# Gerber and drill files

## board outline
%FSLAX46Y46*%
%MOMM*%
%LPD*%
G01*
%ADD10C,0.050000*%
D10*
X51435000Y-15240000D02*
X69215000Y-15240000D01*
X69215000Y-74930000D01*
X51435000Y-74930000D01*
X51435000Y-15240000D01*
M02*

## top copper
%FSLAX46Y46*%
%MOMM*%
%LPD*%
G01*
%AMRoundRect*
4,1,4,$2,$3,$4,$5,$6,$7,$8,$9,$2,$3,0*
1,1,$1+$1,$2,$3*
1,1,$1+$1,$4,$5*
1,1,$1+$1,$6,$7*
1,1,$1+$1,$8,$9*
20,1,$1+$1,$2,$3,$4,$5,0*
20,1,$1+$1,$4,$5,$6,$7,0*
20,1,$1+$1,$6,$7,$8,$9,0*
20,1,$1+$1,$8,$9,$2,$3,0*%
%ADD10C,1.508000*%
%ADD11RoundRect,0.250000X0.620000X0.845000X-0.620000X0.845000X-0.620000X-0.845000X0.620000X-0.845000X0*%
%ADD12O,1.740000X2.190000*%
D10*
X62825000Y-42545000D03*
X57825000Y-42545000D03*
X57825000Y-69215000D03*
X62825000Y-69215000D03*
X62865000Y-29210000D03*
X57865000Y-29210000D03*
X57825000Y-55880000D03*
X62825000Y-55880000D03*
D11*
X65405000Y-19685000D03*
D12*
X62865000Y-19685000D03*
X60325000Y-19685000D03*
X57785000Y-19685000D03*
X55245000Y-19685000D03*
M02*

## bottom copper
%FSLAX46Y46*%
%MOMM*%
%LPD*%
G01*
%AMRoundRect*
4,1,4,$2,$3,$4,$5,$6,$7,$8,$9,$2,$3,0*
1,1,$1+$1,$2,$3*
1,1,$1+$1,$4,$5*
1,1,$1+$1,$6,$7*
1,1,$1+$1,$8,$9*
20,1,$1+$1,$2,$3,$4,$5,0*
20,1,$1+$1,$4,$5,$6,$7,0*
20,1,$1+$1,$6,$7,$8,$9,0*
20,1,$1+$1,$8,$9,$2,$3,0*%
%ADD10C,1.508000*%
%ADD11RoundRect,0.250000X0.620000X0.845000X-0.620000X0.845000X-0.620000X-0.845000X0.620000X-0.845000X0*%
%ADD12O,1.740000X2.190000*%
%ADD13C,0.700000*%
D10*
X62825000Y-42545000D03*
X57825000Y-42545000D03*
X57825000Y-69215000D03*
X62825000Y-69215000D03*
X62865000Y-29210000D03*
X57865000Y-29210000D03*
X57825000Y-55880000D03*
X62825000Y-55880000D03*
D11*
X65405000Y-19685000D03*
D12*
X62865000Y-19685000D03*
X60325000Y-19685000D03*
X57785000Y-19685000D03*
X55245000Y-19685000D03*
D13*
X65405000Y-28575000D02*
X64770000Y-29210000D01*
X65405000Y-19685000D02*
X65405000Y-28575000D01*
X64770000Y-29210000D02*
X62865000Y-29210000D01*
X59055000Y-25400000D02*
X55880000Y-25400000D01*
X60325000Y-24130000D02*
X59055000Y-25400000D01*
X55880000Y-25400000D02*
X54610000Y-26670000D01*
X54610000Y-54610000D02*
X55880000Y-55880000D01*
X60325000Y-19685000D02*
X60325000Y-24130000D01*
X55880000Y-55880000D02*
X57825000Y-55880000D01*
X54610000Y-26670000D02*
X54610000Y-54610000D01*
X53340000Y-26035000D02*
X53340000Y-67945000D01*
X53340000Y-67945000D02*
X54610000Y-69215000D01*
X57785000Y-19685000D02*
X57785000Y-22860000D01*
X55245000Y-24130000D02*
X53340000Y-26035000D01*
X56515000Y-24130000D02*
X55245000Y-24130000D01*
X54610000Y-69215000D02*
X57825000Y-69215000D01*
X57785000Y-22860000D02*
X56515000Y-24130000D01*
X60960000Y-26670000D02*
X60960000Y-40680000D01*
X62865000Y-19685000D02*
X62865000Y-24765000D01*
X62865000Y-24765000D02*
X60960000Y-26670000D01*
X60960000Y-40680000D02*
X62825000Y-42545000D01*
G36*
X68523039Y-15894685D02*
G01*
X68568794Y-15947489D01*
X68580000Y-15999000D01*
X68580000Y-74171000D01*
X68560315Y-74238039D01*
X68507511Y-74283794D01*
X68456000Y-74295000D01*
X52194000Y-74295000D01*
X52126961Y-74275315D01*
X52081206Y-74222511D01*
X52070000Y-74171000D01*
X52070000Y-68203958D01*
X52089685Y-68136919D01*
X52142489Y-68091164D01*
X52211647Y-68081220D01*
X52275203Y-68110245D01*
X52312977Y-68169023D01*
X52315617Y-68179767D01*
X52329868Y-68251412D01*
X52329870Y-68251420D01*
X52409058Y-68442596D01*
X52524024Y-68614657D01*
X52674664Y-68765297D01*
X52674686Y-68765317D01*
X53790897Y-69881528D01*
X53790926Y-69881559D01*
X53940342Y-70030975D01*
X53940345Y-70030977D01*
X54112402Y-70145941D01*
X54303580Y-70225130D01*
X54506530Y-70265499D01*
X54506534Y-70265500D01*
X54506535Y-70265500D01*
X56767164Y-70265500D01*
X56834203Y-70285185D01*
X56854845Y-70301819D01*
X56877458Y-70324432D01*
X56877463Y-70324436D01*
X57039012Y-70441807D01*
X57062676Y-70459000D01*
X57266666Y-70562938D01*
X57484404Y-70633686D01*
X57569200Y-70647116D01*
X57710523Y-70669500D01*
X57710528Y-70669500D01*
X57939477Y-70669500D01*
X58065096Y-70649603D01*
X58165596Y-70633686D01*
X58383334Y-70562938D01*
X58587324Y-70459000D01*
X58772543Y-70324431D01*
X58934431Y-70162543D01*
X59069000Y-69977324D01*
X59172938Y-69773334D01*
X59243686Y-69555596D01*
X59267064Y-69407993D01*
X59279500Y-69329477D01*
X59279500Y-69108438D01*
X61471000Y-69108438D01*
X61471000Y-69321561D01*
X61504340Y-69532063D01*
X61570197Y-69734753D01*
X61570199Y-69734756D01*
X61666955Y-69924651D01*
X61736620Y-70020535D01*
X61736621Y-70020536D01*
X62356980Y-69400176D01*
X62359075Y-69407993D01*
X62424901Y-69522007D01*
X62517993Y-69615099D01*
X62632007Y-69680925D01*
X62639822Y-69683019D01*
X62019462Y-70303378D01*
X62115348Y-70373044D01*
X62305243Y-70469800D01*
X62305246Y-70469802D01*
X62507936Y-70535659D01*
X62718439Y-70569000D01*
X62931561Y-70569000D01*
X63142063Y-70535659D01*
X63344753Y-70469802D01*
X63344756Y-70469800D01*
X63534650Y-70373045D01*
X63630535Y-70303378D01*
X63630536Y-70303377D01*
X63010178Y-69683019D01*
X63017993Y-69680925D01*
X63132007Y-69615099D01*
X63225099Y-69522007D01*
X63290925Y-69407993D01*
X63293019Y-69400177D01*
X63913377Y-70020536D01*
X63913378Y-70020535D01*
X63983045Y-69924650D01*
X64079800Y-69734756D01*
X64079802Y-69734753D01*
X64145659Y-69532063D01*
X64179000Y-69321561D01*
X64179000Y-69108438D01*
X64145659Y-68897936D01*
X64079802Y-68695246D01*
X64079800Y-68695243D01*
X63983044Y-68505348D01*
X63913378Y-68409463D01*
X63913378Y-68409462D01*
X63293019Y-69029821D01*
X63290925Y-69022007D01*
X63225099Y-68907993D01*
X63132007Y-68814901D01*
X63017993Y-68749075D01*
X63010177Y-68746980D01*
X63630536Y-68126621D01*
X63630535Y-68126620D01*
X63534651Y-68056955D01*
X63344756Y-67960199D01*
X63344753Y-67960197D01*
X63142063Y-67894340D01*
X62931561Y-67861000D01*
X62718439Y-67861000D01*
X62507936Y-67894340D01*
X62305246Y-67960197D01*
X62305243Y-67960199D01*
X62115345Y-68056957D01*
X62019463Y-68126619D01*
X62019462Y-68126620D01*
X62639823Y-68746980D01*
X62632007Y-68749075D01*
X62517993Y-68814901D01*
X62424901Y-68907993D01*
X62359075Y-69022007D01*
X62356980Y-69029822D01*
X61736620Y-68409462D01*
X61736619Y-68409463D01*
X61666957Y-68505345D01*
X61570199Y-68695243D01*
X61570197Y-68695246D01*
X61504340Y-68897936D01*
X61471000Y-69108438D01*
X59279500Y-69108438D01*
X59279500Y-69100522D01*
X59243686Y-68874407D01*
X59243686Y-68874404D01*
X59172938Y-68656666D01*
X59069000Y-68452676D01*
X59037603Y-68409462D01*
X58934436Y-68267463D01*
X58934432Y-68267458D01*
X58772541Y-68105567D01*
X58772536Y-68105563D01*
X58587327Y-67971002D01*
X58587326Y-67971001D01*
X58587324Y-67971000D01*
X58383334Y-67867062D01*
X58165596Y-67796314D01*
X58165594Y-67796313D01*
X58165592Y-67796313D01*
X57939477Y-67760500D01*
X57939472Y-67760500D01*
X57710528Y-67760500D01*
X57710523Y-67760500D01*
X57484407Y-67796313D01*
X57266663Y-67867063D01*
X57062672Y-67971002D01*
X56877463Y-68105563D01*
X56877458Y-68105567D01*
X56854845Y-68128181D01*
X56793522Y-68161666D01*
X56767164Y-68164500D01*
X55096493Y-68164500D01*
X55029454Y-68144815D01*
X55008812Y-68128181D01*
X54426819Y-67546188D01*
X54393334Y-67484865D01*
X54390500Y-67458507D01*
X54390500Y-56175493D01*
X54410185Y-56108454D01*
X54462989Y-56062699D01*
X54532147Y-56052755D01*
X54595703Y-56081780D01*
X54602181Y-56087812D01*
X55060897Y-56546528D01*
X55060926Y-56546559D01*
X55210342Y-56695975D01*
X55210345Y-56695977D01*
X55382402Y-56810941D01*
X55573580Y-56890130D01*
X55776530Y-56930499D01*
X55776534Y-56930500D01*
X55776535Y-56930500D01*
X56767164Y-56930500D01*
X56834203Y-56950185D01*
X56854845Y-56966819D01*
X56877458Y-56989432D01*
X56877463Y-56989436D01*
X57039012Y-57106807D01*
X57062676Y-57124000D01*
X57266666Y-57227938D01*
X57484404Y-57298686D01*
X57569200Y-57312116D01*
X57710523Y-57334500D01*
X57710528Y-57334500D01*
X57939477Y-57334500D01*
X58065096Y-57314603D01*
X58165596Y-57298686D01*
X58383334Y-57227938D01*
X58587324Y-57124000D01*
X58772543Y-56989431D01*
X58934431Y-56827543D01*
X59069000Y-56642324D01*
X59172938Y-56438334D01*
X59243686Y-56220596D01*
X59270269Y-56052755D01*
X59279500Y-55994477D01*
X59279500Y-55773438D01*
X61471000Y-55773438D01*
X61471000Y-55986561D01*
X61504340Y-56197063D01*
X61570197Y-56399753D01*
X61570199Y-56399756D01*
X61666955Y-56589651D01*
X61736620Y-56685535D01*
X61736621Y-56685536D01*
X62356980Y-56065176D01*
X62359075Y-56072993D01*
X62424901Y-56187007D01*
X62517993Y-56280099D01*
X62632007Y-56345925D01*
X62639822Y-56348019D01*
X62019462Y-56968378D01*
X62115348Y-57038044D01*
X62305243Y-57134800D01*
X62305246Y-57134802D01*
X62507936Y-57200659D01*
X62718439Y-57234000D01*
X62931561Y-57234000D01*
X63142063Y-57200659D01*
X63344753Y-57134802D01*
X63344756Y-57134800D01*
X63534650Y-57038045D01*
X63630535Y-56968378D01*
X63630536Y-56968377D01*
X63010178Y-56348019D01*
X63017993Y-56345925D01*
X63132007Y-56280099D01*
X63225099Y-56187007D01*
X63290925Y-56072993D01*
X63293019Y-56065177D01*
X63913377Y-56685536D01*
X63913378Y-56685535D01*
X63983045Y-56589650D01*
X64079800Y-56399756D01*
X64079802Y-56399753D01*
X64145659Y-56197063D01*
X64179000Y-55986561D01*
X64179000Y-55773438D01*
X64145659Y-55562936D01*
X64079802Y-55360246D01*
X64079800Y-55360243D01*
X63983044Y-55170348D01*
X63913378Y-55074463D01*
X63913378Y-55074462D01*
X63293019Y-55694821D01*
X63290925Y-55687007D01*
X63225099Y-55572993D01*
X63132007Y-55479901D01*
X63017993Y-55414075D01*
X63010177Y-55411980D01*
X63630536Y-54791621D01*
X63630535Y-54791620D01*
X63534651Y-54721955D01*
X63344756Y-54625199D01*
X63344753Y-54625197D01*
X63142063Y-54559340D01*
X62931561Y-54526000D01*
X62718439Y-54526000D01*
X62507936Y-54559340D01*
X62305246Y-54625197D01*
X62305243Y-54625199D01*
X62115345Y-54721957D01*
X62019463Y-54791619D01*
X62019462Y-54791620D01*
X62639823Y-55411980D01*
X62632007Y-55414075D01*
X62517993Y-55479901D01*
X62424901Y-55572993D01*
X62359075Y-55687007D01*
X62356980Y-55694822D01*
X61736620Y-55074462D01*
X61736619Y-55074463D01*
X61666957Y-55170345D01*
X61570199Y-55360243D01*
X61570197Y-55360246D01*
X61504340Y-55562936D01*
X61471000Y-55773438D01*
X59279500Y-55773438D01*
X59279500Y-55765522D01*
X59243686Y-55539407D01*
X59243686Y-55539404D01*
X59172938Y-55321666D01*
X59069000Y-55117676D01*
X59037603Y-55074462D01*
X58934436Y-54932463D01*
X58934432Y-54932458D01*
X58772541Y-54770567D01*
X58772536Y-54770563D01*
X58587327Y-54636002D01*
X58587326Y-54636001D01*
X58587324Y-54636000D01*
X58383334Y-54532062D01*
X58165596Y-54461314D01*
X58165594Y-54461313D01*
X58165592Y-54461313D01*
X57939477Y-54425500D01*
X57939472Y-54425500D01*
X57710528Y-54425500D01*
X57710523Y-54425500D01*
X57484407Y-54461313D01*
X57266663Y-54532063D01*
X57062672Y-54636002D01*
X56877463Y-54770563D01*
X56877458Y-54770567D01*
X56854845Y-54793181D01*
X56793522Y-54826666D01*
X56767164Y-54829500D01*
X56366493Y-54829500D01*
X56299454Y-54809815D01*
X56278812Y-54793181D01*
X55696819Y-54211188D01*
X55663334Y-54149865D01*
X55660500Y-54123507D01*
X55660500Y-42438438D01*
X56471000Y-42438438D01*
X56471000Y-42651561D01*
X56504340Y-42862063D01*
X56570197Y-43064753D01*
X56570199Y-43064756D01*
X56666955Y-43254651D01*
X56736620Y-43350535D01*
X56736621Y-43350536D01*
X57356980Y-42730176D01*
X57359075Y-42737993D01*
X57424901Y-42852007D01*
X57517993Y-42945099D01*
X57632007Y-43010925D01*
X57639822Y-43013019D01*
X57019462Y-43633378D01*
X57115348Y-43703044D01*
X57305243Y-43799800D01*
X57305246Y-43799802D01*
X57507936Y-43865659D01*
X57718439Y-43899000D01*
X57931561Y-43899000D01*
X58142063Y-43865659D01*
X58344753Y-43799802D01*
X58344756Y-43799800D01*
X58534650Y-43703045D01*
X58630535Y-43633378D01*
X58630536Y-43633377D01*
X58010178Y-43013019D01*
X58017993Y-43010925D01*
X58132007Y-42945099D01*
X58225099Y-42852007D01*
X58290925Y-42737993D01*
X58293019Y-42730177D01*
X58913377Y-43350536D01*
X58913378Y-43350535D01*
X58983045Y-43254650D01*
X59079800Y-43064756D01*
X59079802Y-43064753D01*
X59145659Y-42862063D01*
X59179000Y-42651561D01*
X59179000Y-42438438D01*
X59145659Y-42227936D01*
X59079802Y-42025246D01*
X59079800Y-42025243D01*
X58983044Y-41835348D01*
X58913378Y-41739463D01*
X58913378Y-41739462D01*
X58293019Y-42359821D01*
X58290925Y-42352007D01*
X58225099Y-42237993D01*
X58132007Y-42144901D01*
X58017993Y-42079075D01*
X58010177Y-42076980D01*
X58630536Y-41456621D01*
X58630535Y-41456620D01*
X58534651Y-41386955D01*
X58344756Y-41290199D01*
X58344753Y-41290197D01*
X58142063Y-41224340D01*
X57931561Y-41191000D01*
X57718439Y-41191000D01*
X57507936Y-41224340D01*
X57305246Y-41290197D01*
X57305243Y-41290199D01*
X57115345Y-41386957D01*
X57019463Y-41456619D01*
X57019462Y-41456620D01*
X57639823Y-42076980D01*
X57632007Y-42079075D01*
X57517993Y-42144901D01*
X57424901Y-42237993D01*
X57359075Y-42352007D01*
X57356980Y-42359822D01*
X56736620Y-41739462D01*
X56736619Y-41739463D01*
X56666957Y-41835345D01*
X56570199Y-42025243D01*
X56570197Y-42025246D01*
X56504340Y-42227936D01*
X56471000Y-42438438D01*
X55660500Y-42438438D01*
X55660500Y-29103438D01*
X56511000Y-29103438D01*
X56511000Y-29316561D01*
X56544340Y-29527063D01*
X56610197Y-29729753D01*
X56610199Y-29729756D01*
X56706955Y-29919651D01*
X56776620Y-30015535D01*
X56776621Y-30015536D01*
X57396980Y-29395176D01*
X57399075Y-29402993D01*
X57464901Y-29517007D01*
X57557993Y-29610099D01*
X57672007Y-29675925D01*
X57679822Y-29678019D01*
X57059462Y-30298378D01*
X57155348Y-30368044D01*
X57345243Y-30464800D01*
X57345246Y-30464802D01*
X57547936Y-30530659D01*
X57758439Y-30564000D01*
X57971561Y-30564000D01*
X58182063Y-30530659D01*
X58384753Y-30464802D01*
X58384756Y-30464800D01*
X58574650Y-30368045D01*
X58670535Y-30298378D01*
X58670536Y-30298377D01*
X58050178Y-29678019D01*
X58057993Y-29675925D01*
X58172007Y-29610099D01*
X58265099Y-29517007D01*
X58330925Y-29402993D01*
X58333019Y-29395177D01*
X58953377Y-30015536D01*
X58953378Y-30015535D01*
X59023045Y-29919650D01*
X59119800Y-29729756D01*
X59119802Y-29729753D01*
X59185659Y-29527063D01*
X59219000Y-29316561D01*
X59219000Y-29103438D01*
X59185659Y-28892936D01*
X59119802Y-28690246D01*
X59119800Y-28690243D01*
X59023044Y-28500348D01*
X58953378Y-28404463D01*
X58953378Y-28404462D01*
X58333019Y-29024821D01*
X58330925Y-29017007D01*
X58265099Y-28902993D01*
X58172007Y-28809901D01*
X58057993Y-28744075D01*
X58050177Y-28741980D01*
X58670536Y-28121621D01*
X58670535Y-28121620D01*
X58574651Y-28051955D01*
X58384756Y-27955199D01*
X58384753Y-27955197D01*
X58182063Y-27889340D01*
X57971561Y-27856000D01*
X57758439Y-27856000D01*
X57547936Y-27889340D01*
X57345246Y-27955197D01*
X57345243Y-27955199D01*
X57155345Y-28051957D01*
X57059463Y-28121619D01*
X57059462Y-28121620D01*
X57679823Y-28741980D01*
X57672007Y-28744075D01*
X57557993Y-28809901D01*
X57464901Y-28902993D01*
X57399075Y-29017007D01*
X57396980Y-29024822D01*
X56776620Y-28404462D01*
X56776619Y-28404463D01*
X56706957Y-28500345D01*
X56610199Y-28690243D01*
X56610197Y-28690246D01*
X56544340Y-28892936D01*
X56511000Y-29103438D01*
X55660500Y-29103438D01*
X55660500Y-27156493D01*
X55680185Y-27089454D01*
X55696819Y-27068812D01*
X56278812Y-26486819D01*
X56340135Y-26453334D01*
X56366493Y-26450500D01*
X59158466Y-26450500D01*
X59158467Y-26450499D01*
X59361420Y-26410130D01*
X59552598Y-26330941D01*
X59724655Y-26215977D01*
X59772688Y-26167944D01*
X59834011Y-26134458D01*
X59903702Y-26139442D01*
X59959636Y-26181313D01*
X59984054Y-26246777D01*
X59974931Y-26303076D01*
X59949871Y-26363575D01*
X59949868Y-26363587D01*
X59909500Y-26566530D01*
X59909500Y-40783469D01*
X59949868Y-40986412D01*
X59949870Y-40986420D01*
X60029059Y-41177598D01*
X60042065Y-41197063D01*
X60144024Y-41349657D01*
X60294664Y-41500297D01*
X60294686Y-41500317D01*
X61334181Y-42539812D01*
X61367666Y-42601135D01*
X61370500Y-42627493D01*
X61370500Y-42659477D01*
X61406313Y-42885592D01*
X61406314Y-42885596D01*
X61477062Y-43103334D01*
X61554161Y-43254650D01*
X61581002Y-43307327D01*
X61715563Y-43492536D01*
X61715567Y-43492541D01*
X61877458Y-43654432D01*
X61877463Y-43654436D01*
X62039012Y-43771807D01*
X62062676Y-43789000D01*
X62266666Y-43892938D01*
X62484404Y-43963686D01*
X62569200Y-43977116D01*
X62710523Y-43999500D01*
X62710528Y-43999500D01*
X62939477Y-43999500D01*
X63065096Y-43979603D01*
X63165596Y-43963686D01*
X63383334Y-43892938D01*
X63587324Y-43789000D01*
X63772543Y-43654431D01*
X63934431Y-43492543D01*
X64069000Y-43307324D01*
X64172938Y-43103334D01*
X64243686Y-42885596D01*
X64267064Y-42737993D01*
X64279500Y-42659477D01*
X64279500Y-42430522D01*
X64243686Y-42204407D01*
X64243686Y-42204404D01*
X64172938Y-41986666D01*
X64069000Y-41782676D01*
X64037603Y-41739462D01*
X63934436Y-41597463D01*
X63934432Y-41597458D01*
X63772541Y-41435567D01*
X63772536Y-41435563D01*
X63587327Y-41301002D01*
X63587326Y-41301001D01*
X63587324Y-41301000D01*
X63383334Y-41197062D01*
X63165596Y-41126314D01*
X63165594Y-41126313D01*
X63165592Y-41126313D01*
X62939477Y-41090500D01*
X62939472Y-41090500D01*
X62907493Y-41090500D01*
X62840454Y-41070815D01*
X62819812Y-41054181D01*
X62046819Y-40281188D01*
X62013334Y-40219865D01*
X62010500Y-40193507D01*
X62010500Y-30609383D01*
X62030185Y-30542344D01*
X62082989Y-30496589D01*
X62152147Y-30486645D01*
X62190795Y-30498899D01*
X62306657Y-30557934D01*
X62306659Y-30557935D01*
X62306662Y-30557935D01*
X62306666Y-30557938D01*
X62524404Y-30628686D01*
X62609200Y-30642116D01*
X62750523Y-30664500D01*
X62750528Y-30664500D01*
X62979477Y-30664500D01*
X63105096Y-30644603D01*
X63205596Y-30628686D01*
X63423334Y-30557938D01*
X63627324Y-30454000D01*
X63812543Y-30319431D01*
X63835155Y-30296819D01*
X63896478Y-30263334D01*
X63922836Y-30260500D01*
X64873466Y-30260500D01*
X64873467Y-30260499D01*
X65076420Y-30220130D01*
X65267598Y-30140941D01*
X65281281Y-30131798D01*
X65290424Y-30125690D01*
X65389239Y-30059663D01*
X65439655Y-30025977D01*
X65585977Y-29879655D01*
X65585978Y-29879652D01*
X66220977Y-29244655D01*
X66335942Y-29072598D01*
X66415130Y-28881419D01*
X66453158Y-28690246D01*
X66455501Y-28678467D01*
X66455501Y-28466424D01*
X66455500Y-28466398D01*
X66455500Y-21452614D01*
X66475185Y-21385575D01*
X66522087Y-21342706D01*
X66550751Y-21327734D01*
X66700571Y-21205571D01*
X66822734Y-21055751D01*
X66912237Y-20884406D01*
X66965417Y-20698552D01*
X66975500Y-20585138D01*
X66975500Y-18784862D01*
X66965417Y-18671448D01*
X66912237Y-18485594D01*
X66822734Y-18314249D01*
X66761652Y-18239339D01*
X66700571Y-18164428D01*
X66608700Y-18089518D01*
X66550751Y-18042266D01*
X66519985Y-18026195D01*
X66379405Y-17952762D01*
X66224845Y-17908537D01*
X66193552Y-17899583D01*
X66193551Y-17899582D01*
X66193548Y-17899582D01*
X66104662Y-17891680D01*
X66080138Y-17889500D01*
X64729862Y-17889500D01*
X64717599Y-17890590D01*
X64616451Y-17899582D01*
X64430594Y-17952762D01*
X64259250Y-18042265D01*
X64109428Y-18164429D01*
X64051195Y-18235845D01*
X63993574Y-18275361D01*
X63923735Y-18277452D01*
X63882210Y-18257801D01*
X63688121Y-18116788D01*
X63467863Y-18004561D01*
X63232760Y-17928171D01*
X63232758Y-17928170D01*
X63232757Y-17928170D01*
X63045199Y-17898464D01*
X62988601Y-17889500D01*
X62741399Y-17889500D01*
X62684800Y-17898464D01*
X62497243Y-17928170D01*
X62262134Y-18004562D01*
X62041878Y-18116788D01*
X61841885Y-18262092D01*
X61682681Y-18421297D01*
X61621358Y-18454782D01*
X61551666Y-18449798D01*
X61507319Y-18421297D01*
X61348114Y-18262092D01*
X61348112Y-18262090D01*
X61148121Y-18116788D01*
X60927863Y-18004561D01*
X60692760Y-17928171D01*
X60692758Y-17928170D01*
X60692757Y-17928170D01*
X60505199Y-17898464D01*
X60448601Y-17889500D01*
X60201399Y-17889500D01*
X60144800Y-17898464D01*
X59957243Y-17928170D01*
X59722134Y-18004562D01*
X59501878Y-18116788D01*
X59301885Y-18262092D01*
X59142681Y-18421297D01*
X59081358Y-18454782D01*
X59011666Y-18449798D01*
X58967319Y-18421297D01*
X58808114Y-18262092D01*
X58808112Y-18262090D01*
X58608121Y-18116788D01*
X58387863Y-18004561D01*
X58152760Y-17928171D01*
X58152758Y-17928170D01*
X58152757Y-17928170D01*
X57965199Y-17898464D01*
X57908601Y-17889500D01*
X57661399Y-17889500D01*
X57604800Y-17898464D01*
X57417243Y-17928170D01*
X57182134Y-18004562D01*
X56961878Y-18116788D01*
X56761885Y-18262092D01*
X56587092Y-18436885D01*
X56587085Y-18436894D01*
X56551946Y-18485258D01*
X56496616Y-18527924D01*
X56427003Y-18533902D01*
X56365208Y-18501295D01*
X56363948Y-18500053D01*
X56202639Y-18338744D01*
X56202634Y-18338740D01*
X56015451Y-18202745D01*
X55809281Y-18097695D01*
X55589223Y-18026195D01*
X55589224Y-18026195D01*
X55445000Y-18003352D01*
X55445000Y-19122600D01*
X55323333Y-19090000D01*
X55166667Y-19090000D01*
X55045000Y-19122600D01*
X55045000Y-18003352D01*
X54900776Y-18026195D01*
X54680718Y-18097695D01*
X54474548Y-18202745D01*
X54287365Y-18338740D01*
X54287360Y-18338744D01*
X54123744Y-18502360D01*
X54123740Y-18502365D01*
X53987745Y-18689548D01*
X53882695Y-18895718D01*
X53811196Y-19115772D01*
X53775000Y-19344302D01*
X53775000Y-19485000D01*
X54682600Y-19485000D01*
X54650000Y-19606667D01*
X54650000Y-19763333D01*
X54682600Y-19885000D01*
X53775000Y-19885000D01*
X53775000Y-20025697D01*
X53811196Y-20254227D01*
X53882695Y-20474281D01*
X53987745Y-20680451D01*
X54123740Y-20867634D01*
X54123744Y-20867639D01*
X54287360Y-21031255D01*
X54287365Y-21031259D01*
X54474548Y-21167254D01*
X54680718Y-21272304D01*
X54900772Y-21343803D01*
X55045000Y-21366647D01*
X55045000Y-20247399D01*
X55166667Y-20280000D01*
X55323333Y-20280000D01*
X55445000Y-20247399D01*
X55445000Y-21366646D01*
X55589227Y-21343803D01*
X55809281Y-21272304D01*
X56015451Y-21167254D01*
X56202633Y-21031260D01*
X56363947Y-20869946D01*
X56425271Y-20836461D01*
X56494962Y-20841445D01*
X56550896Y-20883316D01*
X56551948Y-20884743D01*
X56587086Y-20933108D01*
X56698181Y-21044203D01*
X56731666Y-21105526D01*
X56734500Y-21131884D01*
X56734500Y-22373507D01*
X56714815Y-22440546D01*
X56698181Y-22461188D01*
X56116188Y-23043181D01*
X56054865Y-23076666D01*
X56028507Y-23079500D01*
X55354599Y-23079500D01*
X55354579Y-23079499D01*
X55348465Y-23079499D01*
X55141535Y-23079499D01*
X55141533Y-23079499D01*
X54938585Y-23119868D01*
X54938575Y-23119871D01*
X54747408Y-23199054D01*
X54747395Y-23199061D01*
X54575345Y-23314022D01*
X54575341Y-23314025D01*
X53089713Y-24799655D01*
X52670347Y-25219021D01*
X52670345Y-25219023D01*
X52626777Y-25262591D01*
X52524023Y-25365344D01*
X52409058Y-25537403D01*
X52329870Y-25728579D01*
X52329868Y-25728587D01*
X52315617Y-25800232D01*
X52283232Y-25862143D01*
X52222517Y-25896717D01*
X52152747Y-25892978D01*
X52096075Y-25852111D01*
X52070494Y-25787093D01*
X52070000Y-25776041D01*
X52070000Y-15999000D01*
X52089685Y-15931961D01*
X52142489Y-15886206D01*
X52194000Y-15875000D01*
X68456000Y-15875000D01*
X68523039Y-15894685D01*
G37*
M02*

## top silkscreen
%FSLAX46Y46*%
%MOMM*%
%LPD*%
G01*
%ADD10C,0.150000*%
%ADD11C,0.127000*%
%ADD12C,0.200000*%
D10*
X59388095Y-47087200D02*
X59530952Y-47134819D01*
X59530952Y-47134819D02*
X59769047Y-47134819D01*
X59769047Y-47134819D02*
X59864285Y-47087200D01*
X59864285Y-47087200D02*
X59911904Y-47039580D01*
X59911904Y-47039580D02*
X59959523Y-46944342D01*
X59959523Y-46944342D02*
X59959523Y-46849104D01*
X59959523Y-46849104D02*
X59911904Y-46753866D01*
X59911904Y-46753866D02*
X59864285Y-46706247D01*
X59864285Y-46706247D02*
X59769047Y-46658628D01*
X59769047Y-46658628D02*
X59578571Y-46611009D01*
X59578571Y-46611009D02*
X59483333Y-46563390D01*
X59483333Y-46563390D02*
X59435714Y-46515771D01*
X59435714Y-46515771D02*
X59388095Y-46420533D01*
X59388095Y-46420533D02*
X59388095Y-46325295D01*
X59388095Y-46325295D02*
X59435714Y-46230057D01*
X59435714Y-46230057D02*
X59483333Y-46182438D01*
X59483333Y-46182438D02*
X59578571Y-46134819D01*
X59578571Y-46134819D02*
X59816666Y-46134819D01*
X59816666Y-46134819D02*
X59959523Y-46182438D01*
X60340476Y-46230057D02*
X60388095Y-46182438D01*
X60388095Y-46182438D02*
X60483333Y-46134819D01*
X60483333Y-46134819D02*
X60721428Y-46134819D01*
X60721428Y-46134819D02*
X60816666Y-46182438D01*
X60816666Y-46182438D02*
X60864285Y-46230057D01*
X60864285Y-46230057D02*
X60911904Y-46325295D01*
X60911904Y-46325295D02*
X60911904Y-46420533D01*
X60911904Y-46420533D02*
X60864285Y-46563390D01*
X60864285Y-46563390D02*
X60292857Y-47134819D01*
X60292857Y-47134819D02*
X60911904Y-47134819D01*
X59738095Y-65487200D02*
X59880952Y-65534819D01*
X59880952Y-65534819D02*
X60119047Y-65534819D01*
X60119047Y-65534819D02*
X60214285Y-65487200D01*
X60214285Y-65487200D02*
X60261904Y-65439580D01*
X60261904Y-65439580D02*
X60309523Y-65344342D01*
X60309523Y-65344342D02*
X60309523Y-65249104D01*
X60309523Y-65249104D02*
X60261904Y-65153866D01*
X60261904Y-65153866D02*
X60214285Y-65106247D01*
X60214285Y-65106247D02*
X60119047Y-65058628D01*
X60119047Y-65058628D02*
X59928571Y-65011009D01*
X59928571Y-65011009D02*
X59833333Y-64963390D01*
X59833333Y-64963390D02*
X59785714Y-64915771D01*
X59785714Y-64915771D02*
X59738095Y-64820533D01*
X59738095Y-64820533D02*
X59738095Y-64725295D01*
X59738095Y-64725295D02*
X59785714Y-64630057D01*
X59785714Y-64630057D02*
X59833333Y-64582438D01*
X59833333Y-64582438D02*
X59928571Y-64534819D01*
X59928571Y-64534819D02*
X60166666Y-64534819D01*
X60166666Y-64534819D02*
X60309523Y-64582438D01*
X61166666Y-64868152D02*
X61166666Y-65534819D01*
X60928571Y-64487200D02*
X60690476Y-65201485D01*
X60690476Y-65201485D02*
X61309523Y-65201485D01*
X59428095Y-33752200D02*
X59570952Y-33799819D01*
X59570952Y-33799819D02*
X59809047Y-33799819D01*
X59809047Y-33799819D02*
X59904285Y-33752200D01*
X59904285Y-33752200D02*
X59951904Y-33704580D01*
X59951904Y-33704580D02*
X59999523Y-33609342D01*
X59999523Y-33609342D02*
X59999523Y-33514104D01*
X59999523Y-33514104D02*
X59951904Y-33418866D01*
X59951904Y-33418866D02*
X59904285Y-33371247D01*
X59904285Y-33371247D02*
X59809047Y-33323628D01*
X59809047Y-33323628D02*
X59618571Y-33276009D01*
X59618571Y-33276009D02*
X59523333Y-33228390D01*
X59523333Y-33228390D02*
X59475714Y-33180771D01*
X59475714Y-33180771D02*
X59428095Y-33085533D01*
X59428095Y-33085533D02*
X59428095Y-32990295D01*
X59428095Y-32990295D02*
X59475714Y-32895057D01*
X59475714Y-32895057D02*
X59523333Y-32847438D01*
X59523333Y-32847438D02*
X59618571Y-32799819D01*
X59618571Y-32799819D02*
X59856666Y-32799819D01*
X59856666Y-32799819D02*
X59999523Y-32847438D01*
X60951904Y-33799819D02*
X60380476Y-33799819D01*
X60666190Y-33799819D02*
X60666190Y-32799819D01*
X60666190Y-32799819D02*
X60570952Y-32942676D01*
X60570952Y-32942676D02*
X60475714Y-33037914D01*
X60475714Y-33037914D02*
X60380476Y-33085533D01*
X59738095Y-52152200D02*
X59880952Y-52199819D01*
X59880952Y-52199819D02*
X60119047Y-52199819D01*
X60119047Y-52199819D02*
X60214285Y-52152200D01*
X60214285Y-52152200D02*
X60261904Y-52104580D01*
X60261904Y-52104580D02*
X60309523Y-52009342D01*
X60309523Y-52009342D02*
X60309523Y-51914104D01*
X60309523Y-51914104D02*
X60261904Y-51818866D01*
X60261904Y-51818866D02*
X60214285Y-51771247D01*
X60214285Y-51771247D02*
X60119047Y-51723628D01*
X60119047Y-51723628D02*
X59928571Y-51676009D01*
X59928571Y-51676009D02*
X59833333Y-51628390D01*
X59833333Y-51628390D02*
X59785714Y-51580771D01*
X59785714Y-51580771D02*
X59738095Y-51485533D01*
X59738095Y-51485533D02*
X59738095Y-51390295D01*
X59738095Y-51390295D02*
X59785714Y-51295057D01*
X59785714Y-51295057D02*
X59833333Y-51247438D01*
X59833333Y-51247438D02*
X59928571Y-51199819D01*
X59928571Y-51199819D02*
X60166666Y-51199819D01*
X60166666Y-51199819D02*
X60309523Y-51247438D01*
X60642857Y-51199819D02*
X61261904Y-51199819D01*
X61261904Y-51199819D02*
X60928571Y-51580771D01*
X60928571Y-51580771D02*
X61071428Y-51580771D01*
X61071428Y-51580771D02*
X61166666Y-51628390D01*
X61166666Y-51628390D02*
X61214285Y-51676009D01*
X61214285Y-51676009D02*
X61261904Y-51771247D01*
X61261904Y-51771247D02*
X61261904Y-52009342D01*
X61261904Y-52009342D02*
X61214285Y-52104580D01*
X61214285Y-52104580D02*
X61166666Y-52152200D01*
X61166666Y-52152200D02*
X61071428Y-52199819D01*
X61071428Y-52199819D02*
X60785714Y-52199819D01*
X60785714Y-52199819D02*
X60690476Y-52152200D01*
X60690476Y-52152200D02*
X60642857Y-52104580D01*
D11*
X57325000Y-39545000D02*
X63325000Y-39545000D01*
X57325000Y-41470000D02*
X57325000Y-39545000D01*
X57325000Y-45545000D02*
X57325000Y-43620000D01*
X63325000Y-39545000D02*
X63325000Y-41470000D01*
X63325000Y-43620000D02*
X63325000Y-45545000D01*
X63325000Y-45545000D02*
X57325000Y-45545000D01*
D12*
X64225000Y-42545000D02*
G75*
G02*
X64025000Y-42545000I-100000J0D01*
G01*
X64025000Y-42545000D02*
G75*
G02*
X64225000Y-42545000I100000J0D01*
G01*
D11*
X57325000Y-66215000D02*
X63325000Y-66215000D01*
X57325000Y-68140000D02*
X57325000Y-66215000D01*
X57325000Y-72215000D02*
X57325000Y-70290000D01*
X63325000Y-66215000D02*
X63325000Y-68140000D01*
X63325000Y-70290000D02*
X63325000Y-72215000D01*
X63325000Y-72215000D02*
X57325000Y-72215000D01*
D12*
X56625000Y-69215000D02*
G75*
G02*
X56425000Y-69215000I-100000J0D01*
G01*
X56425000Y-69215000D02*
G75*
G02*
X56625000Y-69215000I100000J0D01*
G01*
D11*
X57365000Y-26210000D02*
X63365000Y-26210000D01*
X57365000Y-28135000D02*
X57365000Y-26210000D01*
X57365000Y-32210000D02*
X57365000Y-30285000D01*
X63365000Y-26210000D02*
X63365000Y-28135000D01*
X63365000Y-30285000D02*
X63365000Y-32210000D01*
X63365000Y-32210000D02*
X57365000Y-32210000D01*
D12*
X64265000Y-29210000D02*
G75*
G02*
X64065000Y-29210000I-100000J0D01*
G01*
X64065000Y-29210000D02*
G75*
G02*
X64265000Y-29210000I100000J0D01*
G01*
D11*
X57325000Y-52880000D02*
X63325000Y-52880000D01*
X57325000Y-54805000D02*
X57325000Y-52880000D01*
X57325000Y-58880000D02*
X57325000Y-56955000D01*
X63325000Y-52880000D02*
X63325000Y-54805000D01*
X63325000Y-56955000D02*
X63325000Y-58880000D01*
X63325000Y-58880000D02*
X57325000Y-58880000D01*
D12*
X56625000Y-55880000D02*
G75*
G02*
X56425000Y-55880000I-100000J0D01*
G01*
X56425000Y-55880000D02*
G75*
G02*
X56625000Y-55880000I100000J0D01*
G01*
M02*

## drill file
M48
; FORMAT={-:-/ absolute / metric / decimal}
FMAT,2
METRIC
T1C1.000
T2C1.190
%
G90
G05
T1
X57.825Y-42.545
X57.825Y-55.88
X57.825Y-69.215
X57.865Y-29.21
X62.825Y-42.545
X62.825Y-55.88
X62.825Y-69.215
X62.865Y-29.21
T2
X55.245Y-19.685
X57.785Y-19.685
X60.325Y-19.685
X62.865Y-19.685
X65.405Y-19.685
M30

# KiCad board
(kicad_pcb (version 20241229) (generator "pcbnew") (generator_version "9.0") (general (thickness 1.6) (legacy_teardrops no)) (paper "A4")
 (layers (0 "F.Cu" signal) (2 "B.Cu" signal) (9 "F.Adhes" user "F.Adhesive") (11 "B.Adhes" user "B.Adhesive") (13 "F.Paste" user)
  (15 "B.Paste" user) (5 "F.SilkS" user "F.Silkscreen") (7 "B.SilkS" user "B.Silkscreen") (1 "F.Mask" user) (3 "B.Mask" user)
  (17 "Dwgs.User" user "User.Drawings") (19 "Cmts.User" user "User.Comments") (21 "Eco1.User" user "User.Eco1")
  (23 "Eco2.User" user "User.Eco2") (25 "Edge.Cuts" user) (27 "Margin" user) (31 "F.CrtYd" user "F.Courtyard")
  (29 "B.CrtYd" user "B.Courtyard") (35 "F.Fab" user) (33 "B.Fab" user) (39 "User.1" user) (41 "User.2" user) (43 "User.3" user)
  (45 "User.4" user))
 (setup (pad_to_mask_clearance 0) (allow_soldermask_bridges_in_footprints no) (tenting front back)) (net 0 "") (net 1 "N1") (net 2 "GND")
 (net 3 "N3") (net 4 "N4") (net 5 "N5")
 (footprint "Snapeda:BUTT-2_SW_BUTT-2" (layer "F.Cu") (at 60.325 42.545 180)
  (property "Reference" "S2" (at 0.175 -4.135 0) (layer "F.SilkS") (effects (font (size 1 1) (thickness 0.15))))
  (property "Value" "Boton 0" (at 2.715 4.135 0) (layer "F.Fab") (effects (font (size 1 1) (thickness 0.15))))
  (fp_line (start 3 3) (end -3 3) (stroke (width 0.127) (type solid)) (layer "F.SilkS"))
  (fp_line (start 3 1.075) (end 3 3) (stroke (width 0.127) (type solid)) (layer "F.SilkS"))
  (fp_line (start 3 -3) (end 3 -1.075) (stroke (width 0.127) (type solid)) (layer "F.SilkS"))
  (fp_line (start -3 3) (end -3 1.075) (stroke (width 0.127) (type solid)) (layer "F.SilkS"))
  (fp_line (start -3 -1.075) (end -3 -3) (stroke (width 0.127) (type solid)) (layer "F.SilkS"))
  (fp_line (start -3 -3) (end 3 -3) (stroke (width 0.127) (type solid)) (layer "F.SilkS"))
  (fp_circle (center -3.8 0) (end -3.7 0) (stroke (width 0.2) (type solid)) (fill no) (layer "F.SilkS"))
  (pad "1" thru_hole circle (at -2.5 0 180) (size 1.508 1.508) (drill 1) (layers "*.Cu" "*.Mask") (remove_unused_layers no) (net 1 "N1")
   (solder_mask_margin 0.102))
  (pad "2" thru_hole circle (at 2.5 0 180) (size 1.508 1.508) (drill 1) (layers "*.Cu" "*.Mask") (remove_unused_layers no) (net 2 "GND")
   (solder_mask_margin 0.102)))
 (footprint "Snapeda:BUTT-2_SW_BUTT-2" (layer "F.Cu") (at 60.325 69.215)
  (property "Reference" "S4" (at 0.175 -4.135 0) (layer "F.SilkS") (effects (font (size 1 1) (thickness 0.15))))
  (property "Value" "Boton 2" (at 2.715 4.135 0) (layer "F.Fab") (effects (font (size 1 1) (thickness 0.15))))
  (fp_line (start -3 -3) (end 3 -3) (stroke (width 0.127) (type solid)) (layer "F.SilkS"))
  (fp_line (start -3 -1.075) (end -3 -3) (stroke (width 0.127) (type solid)) (layer "F.SilkS"))
  (fp_line (start -3 3) (end -3 1.075) (stroke (width 0.127) (type solid)) (layer "F.SilkS"))
  (fp_line (start 3 -3) (end 3 -1.075) (stroke (width 0.127) (type solid)) (layer "F.SilkS"))
  (fp_line (start 3 1.075) (end 3 3) (stroke (width 0.127) (type solid)) (layer "F.SilkS"))
  (fp_line (start 3 3) (end -3 3) (stroke (width 0.127) (type solid)) (layer "F.SilkS"))
  (fp_circle (center -3.8 0) (end -3.7 0) (stroke (width 0.2) (type solid)) (fill no) (layer "F.SilkS"))
  (pad "1" thru_hole circle (at -2.5 0) (size 1.508 1.508) (drill 1) (layers "*.Cu" "*.Mask") (remove_unused_layers no) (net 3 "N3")
   (solder_mask_margin 0.102))
  (pad "2" thru_hole circle (at 2.5 0) (size 1.508 1.508) (drill 1) (layers "*.Cu" "*.Mask") (remove_unused_layers no) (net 2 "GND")
   (solder_mask_margin 0.102)))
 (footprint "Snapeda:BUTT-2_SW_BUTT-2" (layer "F.Cu") (at 60.365 29.21 180)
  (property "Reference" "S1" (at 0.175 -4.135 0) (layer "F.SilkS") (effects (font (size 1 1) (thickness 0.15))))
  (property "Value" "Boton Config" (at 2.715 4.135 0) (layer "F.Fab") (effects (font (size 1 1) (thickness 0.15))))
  (fp_line (start 3 3) (end -3 3) (stroke (width 0.127) (type solid)) (layer "F.SilkS"))
  (fp_line (start 3 1.075) (end 3 3) (stroke (width 0.127) (type solid)) (layer "F.SilkS"))
  (fp_line (start 3 -3) (end 3 -1.075) (stroke (width 0.127) (type solid)) (layer "F.SilkS"))
  (fp_line (start -3 3) (end -3 1.075) (stroke (width 0.127) (type solid)) (layer "F.SilkS"))
  (fp_line (start -3 -1.075) (end -3 -3) (stroke (width 0.127) (type solid)) (layer "F.SilkS"))
  (fp_line (start -3 -3) (end 3 -3) (stroke (width 0.127) (type solid)) (layer "F.SilkS"))
  (fp_circle (center -3.8 0) (end -3.7 0) (stroke (width 0.2) (type solid)) (fill no) (layer "F.SilkS"))
  (pad "1" thru_hole circle (at -2.5 0 180) (size 1.508 1.508) (drill 1) (layers "*.Cu" "*.Mask") (remove_unused_layers no) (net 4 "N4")
   (solder_mask_margin 0.102))
  (pad "2" thru_hole circle (at 2.5 0 180) (size 1.508 1.508) (drill 1) (layers "*.Cu" "*.Mask") (remove_unused_layers no) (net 2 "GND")
   (solder_mask_margin 0.102)))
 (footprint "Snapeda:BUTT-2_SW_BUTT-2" (layer "F.Cu") (at 60.325 55.88)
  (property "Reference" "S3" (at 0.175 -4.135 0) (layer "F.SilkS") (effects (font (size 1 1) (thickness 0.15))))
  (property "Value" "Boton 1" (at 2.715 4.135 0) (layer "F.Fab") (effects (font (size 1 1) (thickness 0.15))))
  (fp_line (start -3 -3) (end 3 -3) (stroke (width 0.127) (type solid)) (layer "F.SilkS"))
  (fp_line (start -3 -1.075) (end -3 -3) (stroke (width 0.127) (type solid)) (layer "F.SilkS"))
  (fp_line (start -3 3) (end -3 1.075) (stroke (width 0.127) (type solid)) (layer "F.SilkS"))
  (fp_line (start 3 -3) (end 3 -1.075) (stroke (width 0.127) (type solid)) (layer "F.SilkS"))
  (fp_line (start 3 1.075) (end 3 3) (stroke (width 0.127) (type solid)) (layer "F.SilkS"))
  (fp_line (start 3 3) (end -3 3) (stroke (width 0.127) (type solid)) (layer "F.SilkS"))
  (fp_circle (center -3.8 0) (end -3.7 0) (stroke (width 0.2) (type solid)) (fill no) (layer "F.SilkS"))
  (pad "1" thru_hole circle (at -2.5 0) (size 1.508 1.508) (drill 1) (layers "*.Cu" "*.Mask") (remove_unused_layers no) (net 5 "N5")
   (solder_mask_margin 0.102))
  (pad "2" thru_hole circle (at 2.5 0) (size 1.508 1.508) (drill 1) (layers "*.Cu" "*.Mask") (remove_unused_layers no) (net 2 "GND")
   (solder_mask_margin 0.102)))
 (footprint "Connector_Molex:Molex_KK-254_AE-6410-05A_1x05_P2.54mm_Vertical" (layer "B.Cu") (at 65.405 19.685 180)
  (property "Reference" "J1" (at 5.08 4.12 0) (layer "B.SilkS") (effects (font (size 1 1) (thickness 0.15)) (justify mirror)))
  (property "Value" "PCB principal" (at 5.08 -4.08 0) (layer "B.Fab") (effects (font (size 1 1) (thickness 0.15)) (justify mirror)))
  (pad "1" thru_hole roundrect (at 0 0 180) (size 1.74 2.19) (drill 1.19) (layers "*.Cu" "*.Mask") (remove_unused_layers no)
   (roundrect_rratio 0.143678) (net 4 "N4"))
  (pad "2" thru_hole oval (at 2.54 0 180) (size 1.74 2.19) (drill 1.19) (layers "*.Cu" "*.Mask") (remove_unused_layers no) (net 1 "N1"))
  (pad "3" thru_hole oval (at 5.08 0 180) (size 1.74 2.19) (drill 1.19) (layers "*.Cu" "*.Mask") (remove_unused_layers no) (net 5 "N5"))
  (pad "4" thru_hole oval (at 7.62 0 180) (size 1.74 2.19) (drill 1.19) (layers "*.Cu" "*.Mask") (remove_unused_layers no) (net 3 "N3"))
  (pad "5" thru_hole oval (at 10.16 0 180) (size 1.74 2.19) (drill 1.19) (layers "*.Cu" "*.Mask") (remove_unused_layers no) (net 2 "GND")))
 (gr_rect (start 51.435 15.24) (end 69.215 74.93) (stroke (width 0.05) (type default)) (fill no) (layer "Edge.Cuts"))
 (segment (start 65.405 28.575) (end 64.77 29.21) (width 0.7) (layer "B.Cu") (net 4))
 (segment (start 65.405 19.685) (end 65.405 28.575) (width 0.7) (layer "B.Cu") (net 4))
 (segment (start 64.77 29.21) (end 62.865 29.21) (width 0.7) (layer "B.Cu") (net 4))
 (segment (start 59.055 25.4) (end 55.88 25.4) (width 0.7) (layer "B.Cu") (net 5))
 (segment (start 60.325 24.13) (end 59.055 25.4) (width 0.7) (layer "B.Cu") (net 5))
 (segment (start 55.88 25.4) (end 54.61 26.67) (width 0.7) (layer "B.Cu") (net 5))
 (segment (start 54.61 54.61) (end 55.88 55.88) (width 0.7) (layer "B.Cu") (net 5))
 (segment (start 60.325 19.685) (end 60.325 24.13) (width 0.7) (layer "B.Cu") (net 5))
 (segment (start 55.88 55.88) (end 57.825 55.88) (width 0.7) (layer "B.Cu") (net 5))
 (segment (start 54.61 26.67) (end 54.61 54.61) (width 0.7) (layer "B.Cu") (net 5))
 (segment (start 53.34 26.035) (end 53.34 67.945) (width 0.7) (layer "B.Cu") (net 3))
 (segment (start 53.34 67.945) (end 54.61 69.215) (width 0.7) (layer "B.Cu") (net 3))
 (segment (start 57.785 19.685) (end 57.785 22.86) (width 0.7) (layer "B.Cu") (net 3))
 (segment (start 55.245 24.13) (end 53.34 26.035) (width 0.7) (layer "B.Cu") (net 3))
 (segment (start 56.515 24.13) (end 55.245 24.13) (width 0.7) (layer "B.Cu") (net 3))
 (segment (start 54.61 69.215) (end 57.825 69.215) (width 0.7) (layer "B.Cu") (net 3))
 (segment (start 57.785 22.86) (end 56.515 24.13) (width 0.7) (layer "B.Cu") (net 3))
 (segment (start 60.96 26.67) (end 60.96 40.68) (width 0.7) (layer "B.Cu") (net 1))
 (segment (start 62.865 19.685) (end 62.865 24.765) (width 0.7) (layer "B.Cu") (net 1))
 (segment (start 62.865 24.765) (end 60.96 26.67) (width 0.7) (layer "B.Cu") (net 1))
 (segment (start 60.96 40.68) (end 62.825 42.545) (width 0.7) (layer "B.Cu") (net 1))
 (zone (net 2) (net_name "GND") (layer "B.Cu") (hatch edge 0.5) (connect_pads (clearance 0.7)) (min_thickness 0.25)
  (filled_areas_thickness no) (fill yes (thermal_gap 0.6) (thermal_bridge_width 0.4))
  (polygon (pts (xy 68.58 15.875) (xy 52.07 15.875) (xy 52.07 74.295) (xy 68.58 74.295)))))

